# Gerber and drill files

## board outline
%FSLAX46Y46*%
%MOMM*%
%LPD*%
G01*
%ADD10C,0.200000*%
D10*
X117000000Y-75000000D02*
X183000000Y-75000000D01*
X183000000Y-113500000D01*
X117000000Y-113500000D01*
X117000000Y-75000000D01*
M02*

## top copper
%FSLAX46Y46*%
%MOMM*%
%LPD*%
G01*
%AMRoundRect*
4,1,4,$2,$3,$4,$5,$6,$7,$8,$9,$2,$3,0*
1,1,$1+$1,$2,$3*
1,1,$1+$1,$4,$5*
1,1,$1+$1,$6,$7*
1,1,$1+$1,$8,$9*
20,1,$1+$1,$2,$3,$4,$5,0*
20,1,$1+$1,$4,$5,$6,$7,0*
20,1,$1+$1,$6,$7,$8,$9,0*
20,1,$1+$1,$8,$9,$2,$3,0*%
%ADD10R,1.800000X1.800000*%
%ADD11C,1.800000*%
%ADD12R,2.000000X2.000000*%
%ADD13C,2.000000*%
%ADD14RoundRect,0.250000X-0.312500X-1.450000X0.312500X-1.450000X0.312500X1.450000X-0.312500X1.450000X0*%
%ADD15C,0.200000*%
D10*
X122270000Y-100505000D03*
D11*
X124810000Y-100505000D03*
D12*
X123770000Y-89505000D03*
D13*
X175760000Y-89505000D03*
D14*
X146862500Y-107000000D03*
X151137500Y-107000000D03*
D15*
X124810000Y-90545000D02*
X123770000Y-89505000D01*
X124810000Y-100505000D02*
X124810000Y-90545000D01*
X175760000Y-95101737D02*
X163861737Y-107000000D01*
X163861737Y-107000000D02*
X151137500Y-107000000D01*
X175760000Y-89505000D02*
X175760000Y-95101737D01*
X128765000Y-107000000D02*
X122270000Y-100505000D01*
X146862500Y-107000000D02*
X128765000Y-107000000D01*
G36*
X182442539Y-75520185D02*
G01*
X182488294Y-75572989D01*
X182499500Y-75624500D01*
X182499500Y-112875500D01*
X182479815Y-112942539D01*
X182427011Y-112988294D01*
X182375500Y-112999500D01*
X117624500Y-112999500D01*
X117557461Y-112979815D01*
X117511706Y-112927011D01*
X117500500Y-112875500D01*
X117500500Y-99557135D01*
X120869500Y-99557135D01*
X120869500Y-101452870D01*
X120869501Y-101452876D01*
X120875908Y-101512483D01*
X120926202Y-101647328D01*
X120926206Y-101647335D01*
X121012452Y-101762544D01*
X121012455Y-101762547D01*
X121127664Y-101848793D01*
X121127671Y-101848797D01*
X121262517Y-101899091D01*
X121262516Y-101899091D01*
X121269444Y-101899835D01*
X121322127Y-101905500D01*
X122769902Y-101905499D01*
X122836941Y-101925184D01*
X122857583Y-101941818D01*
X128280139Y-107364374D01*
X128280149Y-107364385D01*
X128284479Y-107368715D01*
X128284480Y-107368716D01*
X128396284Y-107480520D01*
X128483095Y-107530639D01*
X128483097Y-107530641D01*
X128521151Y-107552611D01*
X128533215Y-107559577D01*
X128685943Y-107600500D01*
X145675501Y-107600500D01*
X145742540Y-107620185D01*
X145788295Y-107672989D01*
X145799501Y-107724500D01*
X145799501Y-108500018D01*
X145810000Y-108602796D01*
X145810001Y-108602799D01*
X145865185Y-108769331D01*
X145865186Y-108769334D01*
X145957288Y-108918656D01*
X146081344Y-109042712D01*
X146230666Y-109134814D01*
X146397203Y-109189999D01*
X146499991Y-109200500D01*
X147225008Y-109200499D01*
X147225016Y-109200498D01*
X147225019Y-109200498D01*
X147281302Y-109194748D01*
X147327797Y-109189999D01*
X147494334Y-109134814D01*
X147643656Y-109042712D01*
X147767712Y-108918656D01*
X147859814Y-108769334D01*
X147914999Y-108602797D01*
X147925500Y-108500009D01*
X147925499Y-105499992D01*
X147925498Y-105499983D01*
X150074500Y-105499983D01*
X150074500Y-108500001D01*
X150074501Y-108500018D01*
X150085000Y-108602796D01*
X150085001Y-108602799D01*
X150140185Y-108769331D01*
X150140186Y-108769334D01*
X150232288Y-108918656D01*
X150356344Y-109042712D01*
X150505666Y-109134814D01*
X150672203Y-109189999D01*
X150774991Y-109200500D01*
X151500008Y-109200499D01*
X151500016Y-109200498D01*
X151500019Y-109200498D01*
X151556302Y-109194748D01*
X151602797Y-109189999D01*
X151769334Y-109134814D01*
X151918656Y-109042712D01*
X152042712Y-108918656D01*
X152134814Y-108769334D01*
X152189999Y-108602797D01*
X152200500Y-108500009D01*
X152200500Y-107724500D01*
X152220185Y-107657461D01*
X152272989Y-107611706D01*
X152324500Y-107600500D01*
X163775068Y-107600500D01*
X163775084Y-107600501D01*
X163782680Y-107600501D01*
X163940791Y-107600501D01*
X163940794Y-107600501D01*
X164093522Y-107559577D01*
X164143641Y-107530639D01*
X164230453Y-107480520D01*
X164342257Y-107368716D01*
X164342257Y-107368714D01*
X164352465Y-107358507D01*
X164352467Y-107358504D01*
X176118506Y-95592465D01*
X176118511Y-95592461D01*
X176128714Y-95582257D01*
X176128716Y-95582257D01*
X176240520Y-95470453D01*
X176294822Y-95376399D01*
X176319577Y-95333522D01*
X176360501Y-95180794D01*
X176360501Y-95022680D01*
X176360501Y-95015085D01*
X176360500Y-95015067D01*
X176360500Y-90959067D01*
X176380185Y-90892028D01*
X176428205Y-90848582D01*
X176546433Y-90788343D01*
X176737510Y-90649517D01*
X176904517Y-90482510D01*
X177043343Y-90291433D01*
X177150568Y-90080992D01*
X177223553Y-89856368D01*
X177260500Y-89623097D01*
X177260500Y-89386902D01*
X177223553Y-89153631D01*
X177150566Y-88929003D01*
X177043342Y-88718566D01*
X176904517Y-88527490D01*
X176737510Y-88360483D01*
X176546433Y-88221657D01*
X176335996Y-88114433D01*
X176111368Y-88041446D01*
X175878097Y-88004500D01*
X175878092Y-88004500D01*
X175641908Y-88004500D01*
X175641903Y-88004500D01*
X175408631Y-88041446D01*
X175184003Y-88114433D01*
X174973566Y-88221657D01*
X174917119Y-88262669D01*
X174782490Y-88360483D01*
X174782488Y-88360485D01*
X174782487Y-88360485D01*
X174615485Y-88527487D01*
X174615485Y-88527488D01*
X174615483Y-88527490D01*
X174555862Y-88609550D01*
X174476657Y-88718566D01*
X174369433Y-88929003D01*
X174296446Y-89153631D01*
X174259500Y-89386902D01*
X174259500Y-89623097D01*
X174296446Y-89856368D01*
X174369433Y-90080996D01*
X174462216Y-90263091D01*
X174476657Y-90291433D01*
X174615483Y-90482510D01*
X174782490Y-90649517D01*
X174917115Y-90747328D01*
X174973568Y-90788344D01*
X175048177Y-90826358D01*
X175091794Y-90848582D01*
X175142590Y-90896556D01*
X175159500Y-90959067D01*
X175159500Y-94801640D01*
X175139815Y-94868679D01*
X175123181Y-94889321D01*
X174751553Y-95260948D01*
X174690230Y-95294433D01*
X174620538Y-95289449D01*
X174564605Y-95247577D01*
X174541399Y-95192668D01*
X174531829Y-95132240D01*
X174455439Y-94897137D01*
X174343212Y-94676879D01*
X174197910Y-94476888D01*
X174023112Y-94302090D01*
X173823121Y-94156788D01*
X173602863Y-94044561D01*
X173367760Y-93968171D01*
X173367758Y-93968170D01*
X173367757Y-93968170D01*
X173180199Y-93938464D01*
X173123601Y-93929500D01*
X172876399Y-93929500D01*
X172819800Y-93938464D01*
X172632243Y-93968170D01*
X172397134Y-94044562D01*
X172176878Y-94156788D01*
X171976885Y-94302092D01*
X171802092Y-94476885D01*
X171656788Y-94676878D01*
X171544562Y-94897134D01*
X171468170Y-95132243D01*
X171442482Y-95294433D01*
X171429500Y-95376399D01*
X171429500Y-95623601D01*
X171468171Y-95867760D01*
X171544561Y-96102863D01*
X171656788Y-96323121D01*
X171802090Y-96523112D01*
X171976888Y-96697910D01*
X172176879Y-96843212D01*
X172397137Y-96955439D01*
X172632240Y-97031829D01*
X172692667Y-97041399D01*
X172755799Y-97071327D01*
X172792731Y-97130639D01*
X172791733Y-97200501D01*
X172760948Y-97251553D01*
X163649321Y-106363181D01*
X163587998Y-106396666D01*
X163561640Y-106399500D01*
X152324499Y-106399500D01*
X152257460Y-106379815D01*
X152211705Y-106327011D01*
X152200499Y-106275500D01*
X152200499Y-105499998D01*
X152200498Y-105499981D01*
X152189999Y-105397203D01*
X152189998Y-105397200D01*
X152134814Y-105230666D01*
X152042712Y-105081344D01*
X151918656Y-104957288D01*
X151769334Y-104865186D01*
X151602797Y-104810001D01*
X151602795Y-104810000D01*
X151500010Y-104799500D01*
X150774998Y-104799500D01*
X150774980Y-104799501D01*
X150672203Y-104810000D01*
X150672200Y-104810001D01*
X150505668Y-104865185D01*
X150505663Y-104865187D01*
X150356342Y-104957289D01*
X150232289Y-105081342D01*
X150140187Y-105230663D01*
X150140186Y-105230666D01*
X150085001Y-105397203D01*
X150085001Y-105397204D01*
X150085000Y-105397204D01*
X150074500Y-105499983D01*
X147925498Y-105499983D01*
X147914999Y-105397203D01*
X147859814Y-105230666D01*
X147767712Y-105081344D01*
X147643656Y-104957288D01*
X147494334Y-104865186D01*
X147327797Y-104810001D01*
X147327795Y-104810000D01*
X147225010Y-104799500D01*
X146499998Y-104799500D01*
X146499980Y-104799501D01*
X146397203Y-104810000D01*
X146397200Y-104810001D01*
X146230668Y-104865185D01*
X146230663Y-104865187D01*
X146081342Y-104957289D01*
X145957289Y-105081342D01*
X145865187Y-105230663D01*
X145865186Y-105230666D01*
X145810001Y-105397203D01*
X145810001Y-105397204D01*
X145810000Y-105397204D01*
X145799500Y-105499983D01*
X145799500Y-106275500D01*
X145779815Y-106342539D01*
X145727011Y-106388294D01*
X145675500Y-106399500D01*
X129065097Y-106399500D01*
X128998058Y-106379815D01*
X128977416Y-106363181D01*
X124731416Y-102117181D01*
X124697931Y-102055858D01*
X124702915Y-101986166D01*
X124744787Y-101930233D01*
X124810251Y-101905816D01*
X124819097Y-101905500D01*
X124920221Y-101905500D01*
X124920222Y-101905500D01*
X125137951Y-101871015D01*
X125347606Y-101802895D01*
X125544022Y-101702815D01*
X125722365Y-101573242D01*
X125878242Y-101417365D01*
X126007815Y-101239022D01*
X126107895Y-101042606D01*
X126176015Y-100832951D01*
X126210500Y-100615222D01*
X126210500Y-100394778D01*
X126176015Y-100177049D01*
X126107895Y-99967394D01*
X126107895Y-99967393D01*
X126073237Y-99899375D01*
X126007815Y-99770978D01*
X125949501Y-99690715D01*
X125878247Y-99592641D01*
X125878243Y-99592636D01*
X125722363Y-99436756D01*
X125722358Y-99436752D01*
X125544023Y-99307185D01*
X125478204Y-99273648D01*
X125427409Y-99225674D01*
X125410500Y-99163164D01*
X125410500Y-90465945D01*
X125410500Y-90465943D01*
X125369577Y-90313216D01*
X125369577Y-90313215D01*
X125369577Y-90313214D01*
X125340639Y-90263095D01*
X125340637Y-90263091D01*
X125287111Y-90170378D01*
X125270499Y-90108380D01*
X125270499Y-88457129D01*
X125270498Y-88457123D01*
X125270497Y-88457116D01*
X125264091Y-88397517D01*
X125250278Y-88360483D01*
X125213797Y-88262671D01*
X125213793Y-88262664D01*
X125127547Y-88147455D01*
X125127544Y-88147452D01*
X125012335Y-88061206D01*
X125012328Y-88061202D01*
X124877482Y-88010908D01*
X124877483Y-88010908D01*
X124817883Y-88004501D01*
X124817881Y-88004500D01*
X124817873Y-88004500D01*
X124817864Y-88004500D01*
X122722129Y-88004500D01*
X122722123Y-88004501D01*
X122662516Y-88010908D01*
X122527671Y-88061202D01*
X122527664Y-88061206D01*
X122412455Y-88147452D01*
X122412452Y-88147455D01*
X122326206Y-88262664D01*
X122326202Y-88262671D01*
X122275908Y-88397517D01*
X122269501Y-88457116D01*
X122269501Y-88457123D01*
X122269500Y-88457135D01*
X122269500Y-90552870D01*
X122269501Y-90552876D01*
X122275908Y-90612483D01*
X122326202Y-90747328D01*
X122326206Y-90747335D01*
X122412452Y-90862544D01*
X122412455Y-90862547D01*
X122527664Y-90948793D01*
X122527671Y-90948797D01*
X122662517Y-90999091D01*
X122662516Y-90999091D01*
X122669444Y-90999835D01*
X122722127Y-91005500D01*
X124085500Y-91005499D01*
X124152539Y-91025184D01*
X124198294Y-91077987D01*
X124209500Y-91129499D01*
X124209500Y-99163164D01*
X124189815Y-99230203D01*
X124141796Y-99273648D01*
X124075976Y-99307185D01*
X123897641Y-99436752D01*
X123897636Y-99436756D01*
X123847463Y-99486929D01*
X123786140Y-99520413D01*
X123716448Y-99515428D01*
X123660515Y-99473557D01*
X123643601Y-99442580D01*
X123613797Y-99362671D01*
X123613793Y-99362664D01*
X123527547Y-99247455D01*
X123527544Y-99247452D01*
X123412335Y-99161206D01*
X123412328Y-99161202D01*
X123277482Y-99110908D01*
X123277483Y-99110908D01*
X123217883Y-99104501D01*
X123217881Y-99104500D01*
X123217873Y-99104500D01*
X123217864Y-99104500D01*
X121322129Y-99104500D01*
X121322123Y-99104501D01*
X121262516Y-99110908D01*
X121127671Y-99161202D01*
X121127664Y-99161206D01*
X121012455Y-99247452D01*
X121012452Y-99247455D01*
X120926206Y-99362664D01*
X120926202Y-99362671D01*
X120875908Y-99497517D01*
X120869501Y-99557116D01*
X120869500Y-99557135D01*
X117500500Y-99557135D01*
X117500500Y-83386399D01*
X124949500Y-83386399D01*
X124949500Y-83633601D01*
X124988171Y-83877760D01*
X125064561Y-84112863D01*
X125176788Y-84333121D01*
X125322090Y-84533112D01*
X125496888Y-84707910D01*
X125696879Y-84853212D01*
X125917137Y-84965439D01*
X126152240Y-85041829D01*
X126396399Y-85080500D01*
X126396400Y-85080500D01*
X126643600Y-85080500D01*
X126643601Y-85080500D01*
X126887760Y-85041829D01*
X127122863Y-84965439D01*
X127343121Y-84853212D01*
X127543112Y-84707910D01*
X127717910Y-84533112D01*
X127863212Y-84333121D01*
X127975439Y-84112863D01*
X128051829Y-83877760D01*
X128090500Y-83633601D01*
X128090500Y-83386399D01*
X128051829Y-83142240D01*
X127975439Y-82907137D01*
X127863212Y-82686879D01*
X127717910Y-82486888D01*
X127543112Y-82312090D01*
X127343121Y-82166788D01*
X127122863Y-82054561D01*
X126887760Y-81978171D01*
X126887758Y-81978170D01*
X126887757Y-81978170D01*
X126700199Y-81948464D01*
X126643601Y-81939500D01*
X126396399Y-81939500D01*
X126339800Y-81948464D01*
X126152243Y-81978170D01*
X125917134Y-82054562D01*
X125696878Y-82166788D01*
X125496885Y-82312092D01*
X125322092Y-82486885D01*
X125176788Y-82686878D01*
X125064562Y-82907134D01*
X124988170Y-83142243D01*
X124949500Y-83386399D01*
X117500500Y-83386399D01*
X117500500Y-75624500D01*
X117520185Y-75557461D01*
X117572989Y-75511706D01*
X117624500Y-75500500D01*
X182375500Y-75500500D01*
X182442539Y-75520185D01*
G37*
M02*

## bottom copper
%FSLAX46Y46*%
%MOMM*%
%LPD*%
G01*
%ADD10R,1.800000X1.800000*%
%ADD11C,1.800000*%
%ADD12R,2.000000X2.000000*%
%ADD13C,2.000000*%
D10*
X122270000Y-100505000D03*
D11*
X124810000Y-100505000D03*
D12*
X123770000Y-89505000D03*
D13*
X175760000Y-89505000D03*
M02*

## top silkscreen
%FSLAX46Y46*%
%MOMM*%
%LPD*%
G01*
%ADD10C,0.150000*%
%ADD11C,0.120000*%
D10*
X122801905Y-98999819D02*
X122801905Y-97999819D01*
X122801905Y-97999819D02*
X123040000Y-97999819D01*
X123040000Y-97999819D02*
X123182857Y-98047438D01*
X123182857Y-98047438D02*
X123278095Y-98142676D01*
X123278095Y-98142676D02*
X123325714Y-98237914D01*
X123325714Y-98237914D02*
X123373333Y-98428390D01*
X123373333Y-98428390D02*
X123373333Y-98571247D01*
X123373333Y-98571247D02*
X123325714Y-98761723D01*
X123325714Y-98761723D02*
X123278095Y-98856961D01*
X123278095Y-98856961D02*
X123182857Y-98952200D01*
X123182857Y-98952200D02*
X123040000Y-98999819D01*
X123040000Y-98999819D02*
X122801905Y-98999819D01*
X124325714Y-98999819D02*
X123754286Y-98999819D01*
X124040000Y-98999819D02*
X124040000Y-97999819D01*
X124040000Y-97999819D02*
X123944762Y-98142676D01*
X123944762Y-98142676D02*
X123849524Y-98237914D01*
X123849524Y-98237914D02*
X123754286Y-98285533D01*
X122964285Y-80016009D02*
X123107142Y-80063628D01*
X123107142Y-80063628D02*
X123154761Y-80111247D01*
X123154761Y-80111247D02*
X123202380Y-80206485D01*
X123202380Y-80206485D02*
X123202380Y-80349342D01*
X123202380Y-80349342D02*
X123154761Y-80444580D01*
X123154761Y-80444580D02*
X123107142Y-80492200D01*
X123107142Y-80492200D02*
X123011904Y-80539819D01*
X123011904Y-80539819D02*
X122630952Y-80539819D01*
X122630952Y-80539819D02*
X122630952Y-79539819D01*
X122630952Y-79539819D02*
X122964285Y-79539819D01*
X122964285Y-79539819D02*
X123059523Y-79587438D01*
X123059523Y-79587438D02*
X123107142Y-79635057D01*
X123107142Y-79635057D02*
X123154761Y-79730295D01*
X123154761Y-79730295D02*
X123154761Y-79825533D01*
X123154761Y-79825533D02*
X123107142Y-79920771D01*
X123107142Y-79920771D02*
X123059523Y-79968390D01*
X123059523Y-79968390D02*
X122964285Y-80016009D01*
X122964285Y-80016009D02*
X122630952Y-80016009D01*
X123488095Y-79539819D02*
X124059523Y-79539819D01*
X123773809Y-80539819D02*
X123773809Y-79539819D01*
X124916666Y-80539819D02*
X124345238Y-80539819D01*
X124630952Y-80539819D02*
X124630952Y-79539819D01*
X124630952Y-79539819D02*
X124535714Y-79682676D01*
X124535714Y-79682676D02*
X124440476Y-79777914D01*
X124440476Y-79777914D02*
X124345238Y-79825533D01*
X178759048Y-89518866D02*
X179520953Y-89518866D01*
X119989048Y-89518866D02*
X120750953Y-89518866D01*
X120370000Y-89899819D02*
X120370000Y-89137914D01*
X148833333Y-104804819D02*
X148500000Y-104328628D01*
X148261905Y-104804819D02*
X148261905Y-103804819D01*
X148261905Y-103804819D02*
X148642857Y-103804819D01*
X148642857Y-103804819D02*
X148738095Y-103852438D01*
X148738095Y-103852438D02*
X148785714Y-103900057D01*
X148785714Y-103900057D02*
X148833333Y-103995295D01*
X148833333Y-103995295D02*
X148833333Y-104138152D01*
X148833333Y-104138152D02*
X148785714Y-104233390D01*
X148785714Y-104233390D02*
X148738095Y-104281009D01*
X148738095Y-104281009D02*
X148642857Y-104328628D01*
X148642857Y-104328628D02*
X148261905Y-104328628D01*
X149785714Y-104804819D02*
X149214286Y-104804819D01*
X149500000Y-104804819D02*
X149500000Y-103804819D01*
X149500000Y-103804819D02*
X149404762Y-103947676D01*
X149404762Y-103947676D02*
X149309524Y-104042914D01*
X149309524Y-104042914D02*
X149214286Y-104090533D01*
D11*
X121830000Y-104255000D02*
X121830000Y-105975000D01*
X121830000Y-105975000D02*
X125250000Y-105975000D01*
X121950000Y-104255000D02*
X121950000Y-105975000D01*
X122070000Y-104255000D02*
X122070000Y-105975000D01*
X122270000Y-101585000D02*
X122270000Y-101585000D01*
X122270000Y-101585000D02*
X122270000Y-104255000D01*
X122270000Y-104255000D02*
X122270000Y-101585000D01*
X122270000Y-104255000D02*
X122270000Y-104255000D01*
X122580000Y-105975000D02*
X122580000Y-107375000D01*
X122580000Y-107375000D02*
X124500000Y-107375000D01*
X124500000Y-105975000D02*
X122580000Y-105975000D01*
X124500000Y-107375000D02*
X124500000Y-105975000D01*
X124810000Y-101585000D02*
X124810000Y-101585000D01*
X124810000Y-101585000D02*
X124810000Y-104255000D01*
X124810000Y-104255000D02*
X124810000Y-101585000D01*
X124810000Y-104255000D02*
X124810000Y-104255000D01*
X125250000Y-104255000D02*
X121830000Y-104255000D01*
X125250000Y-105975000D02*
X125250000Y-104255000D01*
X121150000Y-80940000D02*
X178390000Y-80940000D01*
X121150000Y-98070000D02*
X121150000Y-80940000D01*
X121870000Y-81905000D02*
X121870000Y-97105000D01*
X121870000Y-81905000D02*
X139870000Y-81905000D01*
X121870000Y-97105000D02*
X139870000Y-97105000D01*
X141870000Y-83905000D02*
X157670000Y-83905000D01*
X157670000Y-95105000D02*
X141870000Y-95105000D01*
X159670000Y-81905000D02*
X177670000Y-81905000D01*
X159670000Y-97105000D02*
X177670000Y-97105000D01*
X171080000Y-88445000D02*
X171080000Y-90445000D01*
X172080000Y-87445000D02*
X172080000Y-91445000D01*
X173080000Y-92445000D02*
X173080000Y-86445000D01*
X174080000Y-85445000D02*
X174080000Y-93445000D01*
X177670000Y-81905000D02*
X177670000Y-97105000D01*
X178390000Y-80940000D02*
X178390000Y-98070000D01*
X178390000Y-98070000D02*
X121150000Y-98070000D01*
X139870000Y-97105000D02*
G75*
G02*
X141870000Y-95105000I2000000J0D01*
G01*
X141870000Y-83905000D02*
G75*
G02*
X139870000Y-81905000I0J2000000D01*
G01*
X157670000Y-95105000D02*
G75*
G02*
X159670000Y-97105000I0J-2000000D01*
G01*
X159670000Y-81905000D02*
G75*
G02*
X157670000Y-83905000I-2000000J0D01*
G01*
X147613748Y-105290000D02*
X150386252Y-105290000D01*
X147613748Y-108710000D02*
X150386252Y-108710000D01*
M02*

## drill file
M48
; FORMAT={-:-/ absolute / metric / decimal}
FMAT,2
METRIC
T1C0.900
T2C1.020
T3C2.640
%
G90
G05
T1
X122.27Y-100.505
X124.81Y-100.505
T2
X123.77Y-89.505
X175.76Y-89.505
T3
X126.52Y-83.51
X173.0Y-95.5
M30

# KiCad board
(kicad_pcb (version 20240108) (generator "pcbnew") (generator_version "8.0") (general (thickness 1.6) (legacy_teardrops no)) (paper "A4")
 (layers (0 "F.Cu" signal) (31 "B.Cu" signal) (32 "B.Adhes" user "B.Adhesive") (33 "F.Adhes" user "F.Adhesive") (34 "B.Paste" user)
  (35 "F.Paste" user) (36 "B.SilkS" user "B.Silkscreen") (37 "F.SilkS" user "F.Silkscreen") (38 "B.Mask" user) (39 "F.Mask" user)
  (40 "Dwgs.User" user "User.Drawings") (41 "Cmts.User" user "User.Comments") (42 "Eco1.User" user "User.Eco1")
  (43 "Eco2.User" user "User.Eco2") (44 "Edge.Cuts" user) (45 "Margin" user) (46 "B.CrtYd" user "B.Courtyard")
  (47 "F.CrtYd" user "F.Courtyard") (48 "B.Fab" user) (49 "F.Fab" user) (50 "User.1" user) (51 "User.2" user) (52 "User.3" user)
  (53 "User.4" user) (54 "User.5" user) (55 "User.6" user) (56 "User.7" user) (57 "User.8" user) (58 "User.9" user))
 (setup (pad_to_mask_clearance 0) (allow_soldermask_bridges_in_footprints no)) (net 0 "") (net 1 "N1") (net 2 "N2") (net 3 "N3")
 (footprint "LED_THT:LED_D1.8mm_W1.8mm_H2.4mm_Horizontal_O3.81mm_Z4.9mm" (layer "F.Cu") (at 122.27 100.505)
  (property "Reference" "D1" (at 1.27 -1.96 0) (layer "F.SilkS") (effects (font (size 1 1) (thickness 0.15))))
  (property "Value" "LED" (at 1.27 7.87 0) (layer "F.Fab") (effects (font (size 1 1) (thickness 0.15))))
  (fp_line (start -0.44 3.75) (end -0.44 5.47) (stroke (width 0.12) (type solid)) (layer "F.SilkS"))
  (fp_line (start -0.44 5.47) (end 2.98 5.47) (stroke (width 0.12) (type solid)) (layer "F.SilkS"))
  (fp_line (start -0.32 3.75) (end -0.32 5.47) (stroke (width 0.12) (type solid)) (layer "F.SilkS"))
  (fp_line (start -0.2 3.75) (end -0.2 5.47) (stroke (width 0.12) (type solid)) (layer "F.SilkS"))
  (fp_line (start 0 1.08) (end 0 1.08) (stroke (width 0.12) (type solid)) (layer "F.SilkS"))
  (fp_line (start 0 1.08) (end 0 3.75) (stroke (width 0.12) (type solid)) (layer "F.SilkS"))
  (fp_line (start 0 3.75) (end 0 1.08) (stroke (width 0.12) (type solid)) (layer "F.SilkS"))
  (fp_line (start 0 3.75) (end 0 3.75) (stroke (width 0.12) (type solid)) (layer "F.SilkS"))
  (fp_line (start 0.31 5.47) (end 0.31 6.87) (stroke (width 0.12) (type solid)) (layer "F.SilkS"))
  (fp_line (start 0.31 6.87) (end 2.23 6.87) (stroke (width 0.12) (type solid)) (layer "F.SilkS"))
  (fp_line (start 2.23 5.47) (end 0.31 5.47) (stroke (width 0.12) (type solid)) (layer "F.SilkS"))
  (fp_line (start 2.23 6.87) (end 2.23 5.47) (stroke (width 0.12) (type solid)) (layer "F.SilkS"))
  (fp_line (start 2.54 1.08) (end 2.54 1.08) (stroke (width 0.12) (type solid)) (layer "F.SilkS"))
  (fp_line (start 2.54 1.08) (end 2.54 3.75) (stroke (width 0.12) (type solid)) (layer "F.SilkS"))
  (fp_line (start 2.54 3.75) (end 2.54 1.08) (stroke (width 0.12) (type solid)) (layer "F.SilkS"))
  (fp_line (start 2.54 3.75) (end 2.54 3.75) (stroke (width 0.12) (type solid)) (layer "F.SilkS"))
  (fp_line (start 2.98 3.75) (end -0.44 3.75) (stroke (width 0.12) (type solid)) (layer "F.SilkS"))
  (fp_line (start 2.98 5.47) (end 2.98 3.75) (stroke (width 0.12) (type solid)) (layer "F.SilkS"))
  (pad "1" thru_hole rect (at 0 0) (size 1.8 1.8) (drill 0.9) (layers "*.Cu" "*.Mask") (remove_unused_layers no) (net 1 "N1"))
  (pad "2" thru_hole circle (at 2.54 0) (size 1.8 1.8) (drill 0.9) (layers "*.Cu" "*.Mask") (remove_unused_layers no) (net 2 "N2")))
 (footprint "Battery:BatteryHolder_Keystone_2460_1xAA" (layer "F.Cu") (at 123.77 89.505)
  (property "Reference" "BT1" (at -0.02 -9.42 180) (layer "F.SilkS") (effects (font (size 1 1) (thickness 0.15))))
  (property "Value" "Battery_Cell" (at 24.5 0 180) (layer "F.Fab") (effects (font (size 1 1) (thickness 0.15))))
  (fp_line (start -2.62 -8.565) (end 54.62 -8.565) (stroke (width 0.12) (type solid)) (layer "F.SilkS"))
  (fp_line (start -2.62 8.565) (end -2.62 -8.565) (stroke (width 0.12) (type solid)) (layer "F.SilkS"))
  (fp_line (start -1.9 -7.6) (end -1.9 7.6) (stroke (width 0.12) (type solid)) (layer "F.SilkS"))
  (fp_line (start -1.9 -7.6) (end 16.1 -7.6) (stroke (width 0.12) (type solid)) (layer "F.SilkS"))
  (fp_line (start -1.9 7.6) (end 16.1 7.6) (stroke (width 0.12) (type solid)) (layer "F.SilkS"))
  (fp_line (start 18.1 -5.6) (end 33.9 -5.6) (stroke (width 0.12) (type solid)) (layer "F.SilkS"))
  (fp_line (start 33.9 5.6) (end 18.1 5.6) (stroke (width 0.12) (type solid)) (layer "F.SilkS"))
  (fp_line (start 35.9 -7.6) (end 53.9 -7.6) (stroke (width 0.12) (type solid)) (layer "F.SilkS"))
  (fp_line (start 35.9 7.6) (end 53.9 7.6) (stroke (width 0.12) (type solid)) (layer "F.SilkS"))
  (fp_line (start 47.31 -1.06) (end 47.31 0.94) (stroke (width 0.12) (type solid)) (layer "F.SilkS"))
  (fp_line (start 48.31 -2.06) (end 48.31 1.94) (stroke (width 0.12) (type solid)) (layer "F.SilkS"))
  (fp_line (start 49.31 2.94) (end 49.31 -3.06) (stroke (width 0.12) (type solid)) (layer "F.SilkS"))
  (fp_line (start 50.31 -4.06) (end 50.31 3.94) (stroke (width 0.12) (type solid)) (layer "F.SilkS"))
  (fp_line (start 53.9 -7.6) (end 53.9 7.6) (stroke (width 0.12) (type solid)) (layer "F.SilkS"))
  (fp_line (start 54.62 -8.565) (end 54.62 8.565) (stroke (width 0.12) (type solid)) (layer "F.SilkS"))
  (fp_line (start 54.62 8.565) (end -2.62 8.565) (stroke (width 0.12) (type solid)) (layer "F.SilkS"))
  (fp_arc (start 16.1 7.6) (mid 16.685786 6.185786) (end 18.1 5.6) (stroke (width 0.12) (type solid)) (layer "F.SilkS"))
  (fp_arc (start 18.1 -5.6) (mid 16.685786 -6.185786) (end 16.1 -7.6) (stroke (width 0.12) (type solid)) (layer "F.SilkS"))
  (fp_arc (start 33.9 5.6) (mid 35.314214 6.185786) (end 35.9 7.6) (stroke (width 0.12) (type solid)) (layer "F.SilkS"))
  (fp_arc (start 35.9 -7.6) (mid 35.314214 -6.185786) (end 33.9 -5.6) (stroke (width 0.12) (type solid)) (layer "F.SilkS"))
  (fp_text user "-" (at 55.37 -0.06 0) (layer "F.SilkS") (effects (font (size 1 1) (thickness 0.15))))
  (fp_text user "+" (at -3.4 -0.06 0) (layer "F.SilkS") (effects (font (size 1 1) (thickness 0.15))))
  (pad "" np_thru_hole circle (at 2.75 -5.995 90) (size 2.64 2.64) (drill 2.64) (layers "*.Cu" "*.Mask"))
  (pad "" np_thru_hole circle (at 49.23 5.995) (size 2.64 2.64) (drill 2.64) (layers "*.Cu" "*.Mask"))
  (pad "1" thru_hole rect (at 0 0 180) (size 2 2) (drill 1.02) (layers "*.Cu" "*.Mask") (remove_unused_layers no) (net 2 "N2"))
  (pad "2" thru_hole circle (at 51.99 0 180) (size 2 2) (drill 1.02) (layers "*.Cu" "*.Mask") (remove_unused_layers no) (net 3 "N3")))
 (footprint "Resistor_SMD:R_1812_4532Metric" (layer "F.Cu") (at 149 107)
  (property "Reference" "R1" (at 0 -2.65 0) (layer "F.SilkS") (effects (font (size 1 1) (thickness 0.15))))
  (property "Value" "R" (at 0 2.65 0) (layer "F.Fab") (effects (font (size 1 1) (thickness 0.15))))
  (fp_line (start -1.386252 -1.71) (end 1.386252 -1.71) (stroke (width 0.12) (type solid)) (layer "F.SilkS"))
  (fp_line (start -1.386252 1.71) (end 1.386252 1.71) (stroke (width 0.12) (type solid)) (layer "F.SilkS"))
  (pad "1" smd roundrect (at -2.1375 0) (size 1.125 3.4) (layers "F.Cu" "F.Paste" "F.Mask") (roundrect_rratio 0.222222) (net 1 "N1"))
  (pad "2" smd roundrect (at 2.1375 0) (size 1.125 3.4) (layers "F.Cu" "F.Paste" "F.Mask") (roundrect_rratio 0.222222) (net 3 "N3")))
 (gr_rect (start 117 75) (end 183 113.5) (stroke (width 0.2) (type default)) (fill none) (layer "Edge.Cuts"))
 (segment (start 124.81 90.545) (end 123.77 89.505) (width 0.2) (layer "F.Cu") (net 2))
 (segment (start 124.81 100.505) (end 124.81 90.545) (width 0.2) (layer "F.Cu") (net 2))
 (segment (start 175.76 95.101737) (end 163.861737 107) (width 0.2) (layer "F.Cu") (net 3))
 (segment (start 163.861737 107) (end 151.1375 107) (width 0.2) (layer "F.Cu") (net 3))
 (segment (start 175.76 89.505) (end 175.76 95.101737) (width 0.2) (layer "F.Cu") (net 3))
 (segment (start 128.765 107) (end 122.27 100.505) (width 0.2) (layer "F.Cu") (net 1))
 (segment (start 146.8625 107) (end 128.765 107) (width 0.2) (layer "F.Cu") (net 1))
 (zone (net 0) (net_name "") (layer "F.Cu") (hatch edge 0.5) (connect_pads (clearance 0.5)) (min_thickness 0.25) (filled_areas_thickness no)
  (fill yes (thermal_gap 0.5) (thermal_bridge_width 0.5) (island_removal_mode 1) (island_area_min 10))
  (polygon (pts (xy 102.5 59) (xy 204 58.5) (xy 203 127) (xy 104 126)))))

